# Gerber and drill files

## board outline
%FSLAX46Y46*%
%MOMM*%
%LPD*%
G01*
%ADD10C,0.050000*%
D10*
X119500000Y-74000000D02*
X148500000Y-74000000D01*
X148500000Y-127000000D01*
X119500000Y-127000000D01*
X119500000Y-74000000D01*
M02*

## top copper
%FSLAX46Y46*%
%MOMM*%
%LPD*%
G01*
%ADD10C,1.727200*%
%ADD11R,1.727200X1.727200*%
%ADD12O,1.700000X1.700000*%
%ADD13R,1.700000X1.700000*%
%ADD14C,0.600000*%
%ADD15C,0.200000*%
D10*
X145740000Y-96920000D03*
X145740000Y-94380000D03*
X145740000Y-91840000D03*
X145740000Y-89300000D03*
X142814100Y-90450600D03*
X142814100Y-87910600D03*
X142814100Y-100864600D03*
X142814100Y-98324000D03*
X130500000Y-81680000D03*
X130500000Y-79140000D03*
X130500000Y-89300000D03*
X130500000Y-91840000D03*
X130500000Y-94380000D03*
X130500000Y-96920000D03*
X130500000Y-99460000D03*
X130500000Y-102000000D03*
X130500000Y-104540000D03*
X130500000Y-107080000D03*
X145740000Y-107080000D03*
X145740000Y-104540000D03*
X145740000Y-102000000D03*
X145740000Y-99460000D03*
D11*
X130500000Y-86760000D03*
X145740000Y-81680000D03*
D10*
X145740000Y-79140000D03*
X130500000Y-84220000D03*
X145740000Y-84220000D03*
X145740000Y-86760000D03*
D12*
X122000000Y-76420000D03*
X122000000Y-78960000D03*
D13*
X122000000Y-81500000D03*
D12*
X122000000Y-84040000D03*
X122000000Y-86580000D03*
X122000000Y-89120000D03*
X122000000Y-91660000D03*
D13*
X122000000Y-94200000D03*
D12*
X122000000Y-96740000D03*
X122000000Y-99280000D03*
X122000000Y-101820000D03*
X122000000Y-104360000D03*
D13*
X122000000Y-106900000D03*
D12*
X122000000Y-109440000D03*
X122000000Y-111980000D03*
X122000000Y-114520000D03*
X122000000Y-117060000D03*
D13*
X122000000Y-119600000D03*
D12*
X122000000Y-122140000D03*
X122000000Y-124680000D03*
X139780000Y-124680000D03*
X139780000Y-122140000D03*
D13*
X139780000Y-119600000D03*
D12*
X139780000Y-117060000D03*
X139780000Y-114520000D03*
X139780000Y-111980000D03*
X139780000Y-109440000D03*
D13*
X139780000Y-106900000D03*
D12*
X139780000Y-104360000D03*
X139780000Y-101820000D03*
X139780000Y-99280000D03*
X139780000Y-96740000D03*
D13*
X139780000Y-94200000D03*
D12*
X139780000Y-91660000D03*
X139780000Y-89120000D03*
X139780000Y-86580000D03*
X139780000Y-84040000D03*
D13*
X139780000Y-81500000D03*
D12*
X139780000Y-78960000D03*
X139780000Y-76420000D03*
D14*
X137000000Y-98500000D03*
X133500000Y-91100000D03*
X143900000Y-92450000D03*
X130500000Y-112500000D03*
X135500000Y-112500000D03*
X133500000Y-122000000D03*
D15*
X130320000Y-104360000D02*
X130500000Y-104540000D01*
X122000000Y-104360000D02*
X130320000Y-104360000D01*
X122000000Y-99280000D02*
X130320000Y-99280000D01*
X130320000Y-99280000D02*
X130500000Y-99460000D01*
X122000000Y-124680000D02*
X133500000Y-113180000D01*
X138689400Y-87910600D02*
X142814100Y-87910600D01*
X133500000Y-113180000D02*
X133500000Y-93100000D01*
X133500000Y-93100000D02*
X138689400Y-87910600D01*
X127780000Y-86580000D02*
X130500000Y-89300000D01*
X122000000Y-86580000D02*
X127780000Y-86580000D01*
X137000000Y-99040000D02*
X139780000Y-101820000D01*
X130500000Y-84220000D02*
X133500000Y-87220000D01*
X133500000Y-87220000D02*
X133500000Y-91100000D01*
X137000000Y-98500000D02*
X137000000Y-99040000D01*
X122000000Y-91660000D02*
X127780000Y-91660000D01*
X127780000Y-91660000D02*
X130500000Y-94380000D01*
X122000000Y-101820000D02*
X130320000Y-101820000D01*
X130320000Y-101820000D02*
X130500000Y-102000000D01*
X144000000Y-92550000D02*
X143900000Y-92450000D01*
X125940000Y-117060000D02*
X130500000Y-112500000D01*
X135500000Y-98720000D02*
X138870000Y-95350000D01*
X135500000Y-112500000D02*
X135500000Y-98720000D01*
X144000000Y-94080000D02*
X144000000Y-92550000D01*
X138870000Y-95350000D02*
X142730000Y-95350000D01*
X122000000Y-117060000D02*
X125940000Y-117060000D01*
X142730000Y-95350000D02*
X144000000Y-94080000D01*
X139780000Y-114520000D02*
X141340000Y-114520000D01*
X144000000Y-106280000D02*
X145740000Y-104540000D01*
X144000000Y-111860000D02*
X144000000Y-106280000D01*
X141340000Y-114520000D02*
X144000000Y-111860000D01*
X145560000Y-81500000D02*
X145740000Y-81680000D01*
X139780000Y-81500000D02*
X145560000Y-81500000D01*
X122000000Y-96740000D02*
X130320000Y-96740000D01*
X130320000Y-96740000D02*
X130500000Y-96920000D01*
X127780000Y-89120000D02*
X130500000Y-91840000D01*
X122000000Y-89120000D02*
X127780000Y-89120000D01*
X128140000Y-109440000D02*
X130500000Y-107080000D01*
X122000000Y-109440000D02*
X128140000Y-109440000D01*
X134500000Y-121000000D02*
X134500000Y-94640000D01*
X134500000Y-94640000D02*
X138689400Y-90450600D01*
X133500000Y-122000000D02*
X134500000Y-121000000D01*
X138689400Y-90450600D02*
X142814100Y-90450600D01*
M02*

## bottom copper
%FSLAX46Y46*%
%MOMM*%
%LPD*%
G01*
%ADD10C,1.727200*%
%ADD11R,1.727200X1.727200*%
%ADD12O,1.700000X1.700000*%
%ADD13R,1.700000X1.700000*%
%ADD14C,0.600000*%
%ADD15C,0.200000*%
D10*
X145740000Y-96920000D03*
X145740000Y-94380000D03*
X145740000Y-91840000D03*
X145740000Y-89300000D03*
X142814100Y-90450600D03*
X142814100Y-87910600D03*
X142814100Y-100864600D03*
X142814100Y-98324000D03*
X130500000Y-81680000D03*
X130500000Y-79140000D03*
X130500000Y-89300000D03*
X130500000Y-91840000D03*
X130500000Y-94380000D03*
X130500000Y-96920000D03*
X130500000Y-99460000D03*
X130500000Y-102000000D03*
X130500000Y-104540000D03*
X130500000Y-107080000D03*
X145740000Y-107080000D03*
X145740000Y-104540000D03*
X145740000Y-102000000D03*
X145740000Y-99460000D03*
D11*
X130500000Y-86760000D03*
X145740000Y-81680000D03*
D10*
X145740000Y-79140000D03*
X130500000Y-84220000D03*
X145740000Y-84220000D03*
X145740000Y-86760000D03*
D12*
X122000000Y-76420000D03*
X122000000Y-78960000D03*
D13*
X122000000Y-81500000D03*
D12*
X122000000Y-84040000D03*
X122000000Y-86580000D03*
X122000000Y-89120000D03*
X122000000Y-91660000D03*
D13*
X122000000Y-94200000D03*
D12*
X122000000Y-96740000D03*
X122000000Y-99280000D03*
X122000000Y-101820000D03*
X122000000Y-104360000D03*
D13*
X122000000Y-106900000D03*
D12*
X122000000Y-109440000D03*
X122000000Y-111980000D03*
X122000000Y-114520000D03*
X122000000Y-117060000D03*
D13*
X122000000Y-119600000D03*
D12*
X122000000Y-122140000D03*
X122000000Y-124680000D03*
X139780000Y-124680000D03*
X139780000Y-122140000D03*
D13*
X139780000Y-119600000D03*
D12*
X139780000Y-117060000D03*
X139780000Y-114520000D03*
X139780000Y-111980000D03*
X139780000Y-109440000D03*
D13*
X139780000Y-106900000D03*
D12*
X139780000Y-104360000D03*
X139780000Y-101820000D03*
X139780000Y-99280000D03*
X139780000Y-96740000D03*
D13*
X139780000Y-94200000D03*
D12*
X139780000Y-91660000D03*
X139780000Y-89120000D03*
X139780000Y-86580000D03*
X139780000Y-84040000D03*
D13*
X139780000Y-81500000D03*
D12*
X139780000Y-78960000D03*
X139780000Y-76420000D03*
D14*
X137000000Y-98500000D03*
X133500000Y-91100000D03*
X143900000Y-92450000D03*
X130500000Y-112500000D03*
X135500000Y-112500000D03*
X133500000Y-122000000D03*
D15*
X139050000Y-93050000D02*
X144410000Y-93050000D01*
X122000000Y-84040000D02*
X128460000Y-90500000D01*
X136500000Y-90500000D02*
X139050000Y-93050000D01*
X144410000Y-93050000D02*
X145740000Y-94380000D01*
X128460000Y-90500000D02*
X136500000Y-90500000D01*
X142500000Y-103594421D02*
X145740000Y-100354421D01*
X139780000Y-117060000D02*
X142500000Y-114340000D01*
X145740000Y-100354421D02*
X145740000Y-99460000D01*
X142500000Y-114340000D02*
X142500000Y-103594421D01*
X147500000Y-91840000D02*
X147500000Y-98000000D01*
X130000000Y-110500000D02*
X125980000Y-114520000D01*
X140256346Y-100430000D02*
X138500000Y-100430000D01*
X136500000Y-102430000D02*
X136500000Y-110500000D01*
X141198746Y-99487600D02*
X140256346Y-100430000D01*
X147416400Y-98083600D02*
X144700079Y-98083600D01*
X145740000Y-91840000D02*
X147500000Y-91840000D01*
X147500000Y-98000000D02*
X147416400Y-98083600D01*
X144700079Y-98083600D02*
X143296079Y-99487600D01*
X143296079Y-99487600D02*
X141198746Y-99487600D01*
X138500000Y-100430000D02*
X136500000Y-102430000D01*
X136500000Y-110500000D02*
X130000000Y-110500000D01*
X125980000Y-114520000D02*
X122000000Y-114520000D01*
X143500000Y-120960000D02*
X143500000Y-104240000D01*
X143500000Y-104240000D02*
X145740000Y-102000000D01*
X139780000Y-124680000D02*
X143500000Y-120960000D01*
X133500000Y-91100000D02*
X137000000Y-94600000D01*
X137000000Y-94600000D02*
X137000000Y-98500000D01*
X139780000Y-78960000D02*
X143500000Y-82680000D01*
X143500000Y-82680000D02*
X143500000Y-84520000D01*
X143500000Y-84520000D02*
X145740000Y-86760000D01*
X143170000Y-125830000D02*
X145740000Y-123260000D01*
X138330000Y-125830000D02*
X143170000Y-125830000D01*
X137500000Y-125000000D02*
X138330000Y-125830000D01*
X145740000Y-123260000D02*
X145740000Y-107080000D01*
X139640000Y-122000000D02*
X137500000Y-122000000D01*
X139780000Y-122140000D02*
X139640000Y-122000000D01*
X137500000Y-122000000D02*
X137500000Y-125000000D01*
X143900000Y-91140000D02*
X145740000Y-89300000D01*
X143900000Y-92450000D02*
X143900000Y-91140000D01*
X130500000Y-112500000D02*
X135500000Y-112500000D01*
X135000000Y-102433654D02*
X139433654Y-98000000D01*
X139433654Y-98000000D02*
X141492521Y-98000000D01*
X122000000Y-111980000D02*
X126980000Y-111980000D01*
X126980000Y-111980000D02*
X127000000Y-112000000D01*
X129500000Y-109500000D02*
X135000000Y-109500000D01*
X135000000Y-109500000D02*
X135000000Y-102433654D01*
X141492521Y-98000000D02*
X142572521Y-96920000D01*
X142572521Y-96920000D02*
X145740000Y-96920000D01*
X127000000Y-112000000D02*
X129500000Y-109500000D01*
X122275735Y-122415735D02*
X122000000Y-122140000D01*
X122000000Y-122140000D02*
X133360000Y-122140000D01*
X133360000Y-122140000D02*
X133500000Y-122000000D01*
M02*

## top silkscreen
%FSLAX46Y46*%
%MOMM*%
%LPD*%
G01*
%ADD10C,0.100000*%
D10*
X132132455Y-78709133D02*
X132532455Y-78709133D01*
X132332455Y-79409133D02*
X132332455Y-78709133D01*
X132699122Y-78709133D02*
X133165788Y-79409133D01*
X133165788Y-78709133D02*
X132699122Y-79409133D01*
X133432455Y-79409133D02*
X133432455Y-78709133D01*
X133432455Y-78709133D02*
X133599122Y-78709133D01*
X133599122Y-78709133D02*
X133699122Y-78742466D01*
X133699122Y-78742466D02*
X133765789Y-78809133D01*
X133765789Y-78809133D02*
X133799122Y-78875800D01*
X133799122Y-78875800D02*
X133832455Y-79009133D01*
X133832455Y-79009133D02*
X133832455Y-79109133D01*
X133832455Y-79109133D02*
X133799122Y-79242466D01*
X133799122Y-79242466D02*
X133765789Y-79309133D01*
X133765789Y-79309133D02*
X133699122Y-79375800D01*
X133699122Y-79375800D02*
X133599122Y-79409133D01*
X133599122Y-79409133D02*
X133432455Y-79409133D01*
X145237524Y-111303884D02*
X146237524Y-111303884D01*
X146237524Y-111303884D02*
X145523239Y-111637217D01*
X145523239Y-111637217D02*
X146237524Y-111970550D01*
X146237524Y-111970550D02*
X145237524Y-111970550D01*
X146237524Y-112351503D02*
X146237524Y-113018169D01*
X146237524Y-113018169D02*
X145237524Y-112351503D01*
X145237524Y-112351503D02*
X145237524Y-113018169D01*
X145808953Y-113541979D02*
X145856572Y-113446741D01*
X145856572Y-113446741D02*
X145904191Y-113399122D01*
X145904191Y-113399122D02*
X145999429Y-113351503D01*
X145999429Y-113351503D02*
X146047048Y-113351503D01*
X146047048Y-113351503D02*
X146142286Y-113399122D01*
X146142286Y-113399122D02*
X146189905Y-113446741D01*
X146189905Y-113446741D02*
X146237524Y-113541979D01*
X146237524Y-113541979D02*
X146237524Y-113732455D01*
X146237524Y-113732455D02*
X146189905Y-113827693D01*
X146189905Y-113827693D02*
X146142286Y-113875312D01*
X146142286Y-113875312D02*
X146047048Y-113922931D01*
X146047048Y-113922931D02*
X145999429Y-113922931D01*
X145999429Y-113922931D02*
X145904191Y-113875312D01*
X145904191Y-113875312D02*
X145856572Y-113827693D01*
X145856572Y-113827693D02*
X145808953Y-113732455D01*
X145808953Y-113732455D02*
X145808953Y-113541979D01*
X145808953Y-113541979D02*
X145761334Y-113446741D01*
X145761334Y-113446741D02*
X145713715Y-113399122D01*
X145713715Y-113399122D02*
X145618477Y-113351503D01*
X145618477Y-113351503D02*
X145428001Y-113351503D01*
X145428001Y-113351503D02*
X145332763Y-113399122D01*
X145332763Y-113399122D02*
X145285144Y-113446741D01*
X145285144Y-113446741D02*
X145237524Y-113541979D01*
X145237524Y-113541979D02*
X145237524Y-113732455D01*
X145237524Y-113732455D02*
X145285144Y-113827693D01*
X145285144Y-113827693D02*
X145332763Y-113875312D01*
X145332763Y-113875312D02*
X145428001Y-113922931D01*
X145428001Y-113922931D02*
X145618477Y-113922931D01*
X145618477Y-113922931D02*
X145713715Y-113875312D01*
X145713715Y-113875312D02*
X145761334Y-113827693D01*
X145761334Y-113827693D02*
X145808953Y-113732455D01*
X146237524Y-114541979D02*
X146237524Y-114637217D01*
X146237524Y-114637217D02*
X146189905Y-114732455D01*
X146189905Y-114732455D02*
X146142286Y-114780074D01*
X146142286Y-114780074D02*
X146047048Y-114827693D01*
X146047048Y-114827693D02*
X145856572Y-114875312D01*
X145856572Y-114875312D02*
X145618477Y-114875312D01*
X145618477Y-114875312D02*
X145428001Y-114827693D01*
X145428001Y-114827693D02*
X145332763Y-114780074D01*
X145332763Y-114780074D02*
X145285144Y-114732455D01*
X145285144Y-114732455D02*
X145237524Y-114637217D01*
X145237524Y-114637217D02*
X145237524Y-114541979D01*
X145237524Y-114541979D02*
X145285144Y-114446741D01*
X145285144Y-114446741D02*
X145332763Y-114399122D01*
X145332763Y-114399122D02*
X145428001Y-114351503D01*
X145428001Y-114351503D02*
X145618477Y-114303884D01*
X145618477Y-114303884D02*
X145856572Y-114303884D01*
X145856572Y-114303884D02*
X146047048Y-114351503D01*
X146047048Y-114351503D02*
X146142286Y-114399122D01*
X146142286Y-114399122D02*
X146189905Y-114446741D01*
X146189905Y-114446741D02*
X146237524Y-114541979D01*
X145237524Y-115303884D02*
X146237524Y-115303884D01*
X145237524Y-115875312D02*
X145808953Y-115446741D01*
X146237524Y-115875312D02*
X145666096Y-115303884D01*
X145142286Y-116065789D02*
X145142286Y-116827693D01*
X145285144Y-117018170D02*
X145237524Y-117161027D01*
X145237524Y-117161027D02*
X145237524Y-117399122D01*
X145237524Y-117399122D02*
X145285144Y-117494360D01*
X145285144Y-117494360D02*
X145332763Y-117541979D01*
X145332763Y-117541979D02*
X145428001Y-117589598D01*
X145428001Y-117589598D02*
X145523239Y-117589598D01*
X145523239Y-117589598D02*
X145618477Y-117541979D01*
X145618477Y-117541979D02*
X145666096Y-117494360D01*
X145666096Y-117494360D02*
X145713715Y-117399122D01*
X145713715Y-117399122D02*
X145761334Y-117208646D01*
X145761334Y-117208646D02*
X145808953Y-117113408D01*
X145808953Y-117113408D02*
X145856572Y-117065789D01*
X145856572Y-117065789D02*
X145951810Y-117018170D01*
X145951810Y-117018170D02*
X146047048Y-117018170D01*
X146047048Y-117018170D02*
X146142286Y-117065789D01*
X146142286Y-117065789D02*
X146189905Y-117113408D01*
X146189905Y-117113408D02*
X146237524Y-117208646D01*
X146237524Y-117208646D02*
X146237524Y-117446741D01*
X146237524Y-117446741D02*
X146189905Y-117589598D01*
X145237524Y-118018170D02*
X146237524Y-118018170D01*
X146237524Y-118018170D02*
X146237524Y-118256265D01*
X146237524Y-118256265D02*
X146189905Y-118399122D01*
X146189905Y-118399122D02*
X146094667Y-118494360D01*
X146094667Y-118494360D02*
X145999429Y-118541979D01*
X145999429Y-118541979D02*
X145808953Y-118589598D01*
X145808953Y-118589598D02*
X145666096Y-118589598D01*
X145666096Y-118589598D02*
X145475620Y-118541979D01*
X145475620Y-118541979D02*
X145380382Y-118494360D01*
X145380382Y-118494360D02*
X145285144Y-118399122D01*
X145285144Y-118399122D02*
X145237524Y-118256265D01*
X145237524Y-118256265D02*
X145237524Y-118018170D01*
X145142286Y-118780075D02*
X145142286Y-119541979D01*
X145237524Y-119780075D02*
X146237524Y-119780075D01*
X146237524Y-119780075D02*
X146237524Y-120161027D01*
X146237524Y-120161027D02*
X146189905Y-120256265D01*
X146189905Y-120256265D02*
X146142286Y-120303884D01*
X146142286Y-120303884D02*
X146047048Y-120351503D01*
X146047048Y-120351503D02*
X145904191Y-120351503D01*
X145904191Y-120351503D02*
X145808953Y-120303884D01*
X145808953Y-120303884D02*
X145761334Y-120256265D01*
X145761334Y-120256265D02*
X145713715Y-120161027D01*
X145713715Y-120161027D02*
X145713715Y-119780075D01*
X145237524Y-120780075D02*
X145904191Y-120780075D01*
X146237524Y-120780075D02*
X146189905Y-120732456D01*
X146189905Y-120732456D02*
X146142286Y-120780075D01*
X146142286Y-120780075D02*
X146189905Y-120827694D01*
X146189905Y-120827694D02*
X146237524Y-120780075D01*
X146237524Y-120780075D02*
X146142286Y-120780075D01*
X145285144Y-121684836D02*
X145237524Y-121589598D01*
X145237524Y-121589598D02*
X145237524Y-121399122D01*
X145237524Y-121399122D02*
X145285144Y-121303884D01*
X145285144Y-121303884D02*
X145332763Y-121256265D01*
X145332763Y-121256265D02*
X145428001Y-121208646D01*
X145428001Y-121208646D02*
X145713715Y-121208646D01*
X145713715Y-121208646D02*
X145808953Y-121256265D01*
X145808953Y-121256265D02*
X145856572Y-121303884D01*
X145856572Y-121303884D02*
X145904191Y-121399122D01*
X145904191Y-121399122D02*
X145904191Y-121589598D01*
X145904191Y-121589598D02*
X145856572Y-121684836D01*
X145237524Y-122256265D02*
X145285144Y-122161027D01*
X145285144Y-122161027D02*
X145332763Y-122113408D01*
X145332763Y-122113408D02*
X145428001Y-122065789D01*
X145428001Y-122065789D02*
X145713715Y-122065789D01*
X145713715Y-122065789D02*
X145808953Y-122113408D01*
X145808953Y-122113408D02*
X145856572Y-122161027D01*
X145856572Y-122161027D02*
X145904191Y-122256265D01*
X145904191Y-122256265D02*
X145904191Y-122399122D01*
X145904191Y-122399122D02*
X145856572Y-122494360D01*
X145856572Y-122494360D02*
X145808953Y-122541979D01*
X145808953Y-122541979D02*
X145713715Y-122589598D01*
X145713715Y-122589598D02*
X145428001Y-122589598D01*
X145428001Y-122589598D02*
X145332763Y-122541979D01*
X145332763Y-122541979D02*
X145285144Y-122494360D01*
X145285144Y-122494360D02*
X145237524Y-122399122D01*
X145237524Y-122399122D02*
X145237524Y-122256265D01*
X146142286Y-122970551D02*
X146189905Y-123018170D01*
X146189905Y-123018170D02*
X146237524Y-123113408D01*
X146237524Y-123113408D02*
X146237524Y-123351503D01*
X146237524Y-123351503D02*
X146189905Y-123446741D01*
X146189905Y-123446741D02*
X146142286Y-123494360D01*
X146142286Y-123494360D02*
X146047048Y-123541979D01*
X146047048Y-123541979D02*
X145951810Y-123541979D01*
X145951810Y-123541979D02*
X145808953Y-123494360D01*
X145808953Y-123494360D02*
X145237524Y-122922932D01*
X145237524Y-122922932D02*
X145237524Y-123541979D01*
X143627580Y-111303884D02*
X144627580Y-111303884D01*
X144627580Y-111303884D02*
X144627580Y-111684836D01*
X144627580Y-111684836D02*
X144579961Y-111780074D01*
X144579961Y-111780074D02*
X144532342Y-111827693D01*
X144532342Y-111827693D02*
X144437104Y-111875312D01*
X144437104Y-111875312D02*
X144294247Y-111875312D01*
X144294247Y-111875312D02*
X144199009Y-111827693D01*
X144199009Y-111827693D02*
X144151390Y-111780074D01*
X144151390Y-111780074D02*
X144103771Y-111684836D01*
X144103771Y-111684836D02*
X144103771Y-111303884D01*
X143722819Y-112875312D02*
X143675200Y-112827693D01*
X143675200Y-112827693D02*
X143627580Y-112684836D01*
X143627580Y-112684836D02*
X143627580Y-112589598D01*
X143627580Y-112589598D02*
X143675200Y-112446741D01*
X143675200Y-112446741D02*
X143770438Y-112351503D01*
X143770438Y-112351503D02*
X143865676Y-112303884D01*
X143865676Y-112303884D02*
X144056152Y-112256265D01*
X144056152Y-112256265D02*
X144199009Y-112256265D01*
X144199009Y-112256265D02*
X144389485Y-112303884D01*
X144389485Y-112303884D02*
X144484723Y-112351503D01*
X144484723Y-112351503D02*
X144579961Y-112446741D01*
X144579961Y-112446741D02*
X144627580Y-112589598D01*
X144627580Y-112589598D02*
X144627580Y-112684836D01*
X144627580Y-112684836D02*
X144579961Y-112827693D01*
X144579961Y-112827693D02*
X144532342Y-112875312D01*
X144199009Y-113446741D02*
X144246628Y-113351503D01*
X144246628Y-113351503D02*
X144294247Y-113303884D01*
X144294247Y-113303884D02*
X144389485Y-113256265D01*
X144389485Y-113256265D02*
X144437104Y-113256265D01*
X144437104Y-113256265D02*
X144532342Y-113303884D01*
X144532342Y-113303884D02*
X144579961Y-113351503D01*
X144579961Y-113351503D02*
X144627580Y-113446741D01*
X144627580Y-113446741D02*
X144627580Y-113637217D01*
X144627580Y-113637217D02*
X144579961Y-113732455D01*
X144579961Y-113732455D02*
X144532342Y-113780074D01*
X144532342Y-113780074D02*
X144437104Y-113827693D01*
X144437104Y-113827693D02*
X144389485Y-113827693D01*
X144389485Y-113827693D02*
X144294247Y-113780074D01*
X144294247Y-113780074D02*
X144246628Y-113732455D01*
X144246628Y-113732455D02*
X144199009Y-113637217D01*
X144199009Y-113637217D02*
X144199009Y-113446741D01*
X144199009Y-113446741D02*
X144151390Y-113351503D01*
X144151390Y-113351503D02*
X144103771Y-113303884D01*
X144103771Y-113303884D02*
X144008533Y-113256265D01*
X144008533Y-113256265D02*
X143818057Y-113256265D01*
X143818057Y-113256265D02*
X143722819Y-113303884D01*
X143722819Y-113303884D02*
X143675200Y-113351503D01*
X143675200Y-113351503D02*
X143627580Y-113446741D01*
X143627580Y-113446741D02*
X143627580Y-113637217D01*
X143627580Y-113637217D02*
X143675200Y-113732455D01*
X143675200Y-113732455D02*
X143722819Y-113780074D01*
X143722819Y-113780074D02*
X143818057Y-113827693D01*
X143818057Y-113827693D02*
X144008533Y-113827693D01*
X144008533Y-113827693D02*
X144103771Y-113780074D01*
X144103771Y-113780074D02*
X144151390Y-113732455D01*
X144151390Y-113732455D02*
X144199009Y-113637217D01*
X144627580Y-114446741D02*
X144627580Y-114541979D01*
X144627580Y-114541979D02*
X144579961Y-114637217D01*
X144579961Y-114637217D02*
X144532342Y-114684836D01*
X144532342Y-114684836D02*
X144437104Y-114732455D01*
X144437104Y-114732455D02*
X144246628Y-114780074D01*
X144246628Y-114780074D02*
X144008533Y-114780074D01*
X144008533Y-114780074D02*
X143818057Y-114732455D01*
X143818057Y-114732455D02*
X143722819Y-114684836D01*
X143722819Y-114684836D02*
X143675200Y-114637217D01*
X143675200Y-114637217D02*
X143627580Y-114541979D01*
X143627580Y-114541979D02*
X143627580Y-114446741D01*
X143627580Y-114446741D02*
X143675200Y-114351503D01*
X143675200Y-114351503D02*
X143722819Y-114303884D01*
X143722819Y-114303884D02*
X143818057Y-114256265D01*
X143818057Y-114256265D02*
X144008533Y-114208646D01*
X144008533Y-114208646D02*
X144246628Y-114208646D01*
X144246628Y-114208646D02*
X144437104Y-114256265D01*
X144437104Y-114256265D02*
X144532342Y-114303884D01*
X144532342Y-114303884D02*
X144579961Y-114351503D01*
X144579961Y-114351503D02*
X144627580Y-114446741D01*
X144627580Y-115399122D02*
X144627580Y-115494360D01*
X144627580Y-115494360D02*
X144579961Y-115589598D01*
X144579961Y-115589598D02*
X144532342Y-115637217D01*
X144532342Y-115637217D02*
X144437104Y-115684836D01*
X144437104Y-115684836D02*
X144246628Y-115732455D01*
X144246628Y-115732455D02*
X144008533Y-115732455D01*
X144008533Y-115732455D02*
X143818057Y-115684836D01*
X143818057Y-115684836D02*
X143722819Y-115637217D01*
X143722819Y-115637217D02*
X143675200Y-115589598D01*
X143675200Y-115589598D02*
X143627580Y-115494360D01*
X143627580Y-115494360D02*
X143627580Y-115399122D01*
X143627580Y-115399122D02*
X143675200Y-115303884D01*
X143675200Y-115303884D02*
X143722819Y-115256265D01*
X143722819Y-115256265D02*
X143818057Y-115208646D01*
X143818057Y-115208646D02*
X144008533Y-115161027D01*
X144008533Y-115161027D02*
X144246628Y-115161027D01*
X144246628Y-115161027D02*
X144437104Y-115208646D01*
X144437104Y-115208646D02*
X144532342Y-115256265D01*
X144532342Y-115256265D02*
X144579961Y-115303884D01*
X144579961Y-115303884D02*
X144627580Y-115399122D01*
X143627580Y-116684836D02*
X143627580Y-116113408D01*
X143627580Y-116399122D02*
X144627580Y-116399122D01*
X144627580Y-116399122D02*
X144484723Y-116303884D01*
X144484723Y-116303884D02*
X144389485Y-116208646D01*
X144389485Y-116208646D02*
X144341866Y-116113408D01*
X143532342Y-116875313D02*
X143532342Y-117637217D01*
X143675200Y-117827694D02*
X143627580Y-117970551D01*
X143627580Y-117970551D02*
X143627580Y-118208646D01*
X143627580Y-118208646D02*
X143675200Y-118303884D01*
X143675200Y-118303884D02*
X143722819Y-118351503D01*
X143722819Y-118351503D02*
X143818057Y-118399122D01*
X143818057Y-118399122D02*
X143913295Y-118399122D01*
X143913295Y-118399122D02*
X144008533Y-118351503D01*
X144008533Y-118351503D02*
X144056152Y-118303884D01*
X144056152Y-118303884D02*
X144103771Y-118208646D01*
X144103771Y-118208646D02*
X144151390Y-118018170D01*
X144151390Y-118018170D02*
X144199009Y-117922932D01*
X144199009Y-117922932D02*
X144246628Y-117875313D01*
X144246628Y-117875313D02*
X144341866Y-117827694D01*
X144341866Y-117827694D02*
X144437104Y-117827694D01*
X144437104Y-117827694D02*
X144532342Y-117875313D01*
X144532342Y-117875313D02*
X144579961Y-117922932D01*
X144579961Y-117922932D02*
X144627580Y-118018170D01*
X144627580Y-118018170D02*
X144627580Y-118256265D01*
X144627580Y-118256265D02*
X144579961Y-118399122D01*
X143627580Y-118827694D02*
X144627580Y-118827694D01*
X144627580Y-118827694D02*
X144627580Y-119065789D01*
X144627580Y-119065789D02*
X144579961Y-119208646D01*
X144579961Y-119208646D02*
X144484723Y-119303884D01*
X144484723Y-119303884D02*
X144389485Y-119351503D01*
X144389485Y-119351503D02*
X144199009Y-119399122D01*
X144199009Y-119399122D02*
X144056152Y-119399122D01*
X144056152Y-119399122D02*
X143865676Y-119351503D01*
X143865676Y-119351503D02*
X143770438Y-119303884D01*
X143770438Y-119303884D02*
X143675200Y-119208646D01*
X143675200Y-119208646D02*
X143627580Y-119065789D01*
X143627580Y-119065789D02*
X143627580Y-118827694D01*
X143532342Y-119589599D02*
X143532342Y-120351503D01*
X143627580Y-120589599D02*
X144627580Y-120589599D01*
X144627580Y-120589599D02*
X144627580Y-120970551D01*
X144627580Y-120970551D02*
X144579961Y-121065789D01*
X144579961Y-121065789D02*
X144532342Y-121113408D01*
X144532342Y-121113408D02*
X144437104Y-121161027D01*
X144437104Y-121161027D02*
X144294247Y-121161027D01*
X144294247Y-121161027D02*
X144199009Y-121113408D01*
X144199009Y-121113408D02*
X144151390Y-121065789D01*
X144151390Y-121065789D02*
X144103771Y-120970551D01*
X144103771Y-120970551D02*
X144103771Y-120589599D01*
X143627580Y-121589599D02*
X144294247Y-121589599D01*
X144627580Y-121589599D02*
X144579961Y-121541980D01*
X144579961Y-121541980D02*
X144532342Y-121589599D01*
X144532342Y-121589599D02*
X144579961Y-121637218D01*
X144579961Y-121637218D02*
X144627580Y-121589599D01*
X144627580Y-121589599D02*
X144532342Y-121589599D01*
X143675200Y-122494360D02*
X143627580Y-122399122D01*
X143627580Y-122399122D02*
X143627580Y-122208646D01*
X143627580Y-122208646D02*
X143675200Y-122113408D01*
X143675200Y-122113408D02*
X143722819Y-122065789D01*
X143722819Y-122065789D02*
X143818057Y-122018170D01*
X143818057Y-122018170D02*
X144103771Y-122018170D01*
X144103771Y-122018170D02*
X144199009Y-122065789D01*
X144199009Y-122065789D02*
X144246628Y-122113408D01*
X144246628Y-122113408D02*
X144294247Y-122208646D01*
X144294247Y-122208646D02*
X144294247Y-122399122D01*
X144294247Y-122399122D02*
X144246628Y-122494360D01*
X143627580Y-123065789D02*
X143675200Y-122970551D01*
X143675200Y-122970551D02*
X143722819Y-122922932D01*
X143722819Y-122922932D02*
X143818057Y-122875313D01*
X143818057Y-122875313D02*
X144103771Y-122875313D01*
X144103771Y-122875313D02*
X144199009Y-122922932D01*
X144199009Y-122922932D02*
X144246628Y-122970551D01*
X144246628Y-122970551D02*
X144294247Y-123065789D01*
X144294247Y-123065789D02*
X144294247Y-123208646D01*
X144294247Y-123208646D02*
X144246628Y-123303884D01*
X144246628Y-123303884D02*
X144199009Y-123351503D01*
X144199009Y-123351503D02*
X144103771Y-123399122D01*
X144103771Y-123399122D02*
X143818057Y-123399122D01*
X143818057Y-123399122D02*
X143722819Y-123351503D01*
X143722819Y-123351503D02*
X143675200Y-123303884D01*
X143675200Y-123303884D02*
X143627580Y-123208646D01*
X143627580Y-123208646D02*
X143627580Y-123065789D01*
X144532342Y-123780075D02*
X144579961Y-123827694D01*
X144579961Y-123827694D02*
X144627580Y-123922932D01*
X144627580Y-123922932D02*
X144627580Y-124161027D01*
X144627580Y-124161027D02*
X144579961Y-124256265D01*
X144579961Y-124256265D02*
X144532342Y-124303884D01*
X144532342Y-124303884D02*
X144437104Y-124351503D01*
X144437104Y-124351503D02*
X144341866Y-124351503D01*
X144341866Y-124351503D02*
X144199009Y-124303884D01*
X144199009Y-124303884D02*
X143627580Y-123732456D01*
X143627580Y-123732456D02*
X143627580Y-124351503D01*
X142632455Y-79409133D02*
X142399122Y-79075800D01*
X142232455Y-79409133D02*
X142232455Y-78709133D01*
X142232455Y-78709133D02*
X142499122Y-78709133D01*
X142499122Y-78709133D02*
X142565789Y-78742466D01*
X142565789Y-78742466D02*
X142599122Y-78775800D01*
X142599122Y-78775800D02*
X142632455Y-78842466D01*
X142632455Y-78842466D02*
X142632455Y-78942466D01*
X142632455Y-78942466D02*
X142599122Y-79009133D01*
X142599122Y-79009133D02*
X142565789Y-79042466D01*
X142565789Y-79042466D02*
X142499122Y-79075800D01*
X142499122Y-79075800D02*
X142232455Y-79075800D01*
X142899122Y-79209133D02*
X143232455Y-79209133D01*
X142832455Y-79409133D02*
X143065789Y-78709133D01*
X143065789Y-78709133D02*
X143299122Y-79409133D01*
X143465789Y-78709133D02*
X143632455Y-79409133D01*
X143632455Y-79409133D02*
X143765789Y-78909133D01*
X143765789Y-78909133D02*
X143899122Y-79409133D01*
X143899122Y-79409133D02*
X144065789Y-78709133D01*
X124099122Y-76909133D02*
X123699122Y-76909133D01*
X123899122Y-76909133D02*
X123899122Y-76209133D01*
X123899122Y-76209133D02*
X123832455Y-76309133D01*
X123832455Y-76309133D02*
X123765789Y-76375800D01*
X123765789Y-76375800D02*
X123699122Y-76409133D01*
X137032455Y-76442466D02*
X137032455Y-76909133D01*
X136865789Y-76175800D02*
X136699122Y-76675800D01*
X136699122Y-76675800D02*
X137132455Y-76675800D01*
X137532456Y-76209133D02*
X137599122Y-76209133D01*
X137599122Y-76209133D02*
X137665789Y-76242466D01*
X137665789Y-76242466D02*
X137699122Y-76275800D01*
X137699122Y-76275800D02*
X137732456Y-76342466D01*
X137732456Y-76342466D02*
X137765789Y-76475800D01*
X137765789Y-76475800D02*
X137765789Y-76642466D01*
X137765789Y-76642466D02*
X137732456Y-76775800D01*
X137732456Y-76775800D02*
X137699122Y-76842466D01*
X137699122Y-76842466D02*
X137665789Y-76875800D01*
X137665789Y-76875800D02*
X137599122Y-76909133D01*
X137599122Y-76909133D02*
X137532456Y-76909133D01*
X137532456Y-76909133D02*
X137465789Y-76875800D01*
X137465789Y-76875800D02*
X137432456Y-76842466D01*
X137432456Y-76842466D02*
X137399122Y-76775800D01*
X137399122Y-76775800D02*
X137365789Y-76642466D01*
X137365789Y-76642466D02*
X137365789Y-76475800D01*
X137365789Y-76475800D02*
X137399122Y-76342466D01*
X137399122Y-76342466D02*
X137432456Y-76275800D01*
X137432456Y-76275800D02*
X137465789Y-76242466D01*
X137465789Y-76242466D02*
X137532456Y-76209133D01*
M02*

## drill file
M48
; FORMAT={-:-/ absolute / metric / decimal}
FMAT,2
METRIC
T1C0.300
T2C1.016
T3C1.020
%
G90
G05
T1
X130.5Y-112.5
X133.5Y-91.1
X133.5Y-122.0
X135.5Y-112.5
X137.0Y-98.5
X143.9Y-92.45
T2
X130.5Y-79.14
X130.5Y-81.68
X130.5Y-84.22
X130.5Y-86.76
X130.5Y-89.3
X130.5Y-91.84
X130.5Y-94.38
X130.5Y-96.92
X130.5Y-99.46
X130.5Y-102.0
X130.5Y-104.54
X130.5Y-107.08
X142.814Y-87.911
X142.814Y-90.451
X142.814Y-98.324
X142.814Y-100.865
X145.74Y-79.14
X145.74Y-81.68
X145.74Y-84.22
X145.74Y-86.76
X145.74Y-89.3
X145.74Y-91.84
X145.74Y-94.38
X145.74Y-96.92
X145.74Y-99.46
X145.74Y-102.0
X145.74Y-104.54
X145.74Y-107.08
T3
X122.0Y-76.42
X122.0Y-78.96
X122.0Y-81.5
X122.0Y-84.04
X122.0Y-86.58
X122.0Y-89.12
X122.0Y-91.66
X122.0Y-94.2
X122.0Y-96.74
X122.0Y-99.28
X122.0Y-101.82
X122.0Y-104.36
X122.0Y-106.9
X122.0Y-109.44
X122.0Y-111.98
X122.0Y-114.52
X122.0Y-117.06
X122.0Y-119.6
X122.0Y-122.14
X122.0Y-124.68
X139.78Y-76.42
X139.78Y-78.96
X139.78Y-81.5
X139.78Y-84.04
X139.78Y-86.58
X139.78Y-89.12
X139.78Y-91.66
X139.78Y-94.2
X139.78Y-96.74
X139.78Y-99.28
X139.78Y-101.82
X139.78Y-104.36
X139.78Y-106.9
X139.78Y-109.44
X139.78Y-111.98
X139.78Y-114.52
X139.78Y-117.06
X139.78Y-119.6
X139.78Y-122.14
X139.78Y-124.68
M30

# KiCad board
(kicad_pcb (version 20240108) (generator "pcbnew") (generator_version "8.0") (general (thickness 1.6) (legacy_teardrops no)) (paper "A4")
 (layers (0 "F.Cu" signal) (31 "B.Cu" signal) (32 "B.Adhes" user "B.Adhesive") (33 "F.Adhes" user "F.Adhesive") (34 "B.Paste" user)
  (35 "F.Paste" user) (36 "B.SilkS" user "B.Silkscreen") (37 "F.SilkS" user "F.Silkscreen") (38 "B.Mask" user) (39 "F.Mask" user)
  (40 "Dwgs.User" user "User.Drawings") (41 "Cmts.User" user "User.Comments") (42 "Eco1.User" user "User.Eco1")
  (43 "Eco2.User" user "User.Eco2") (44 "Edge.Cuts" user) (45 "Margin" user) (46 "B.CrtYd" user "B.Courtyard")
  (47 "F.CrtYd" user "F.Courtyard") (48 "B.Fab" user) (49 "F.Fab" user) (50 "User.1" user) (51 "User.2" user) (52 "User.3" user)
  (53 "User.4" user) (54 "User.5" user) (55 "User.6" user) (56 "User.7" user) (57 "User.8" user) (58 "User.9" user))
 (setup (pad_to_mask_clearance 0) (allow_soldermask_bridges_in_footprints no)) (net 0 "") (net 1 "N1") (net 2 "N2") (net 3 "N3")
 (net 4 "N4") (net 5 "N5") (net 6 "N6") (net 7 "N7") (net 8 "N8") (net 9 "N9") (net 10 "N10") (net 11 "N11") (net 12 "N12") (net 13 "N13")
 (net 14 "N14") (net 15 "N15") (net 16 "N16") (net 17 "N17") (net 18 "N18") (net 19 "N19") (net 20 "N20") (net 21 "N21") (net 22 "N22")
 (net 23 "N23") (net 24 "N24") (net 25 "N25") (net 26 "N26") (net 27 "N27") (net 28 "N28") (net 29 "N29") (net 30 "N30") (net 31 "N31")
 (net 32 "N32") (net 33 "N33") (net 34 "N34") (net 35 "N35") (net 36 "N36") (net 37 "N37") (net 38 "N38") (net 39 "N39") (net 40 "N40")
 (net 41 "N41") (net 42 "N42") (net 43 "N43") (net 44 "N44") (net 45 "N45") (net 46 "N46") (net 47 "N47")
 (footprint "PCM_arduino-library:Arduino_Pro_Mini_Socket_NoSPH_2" (layer "F.Cu") (at 138.12 91.84)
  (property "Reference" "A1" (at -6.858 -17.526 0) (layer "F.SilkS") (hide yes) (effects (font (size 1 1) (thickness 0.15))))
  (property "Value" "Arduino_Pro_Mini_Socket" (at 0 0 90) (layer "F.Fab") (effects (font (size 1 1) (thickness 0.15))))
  (pad "A0" thru_hole circle (at 7.62 5.08) (size 1.7272 1.7272) (drill 1.016) (layers "*.Cu" "*.Mask") (remove_unused_layers no)
   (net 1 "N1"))
  (pad "A1" thru_hole circle (at 7.62 2.54) (size 1.7272 1.7272) (drill 1.016) (layers "*.Cu" "*.Mask") (remove_unused_layers no)
   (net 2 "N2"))
  (pad "A2" thru_hole circle (at 7.62 0) (size 1.7272 1.7272) (drill 1.016) (layers "*.Cu" "*.Mask") (remove_unused_layers no) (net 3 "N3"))
  (pad "A3" thru_hole circle (at 7.62 -2.54) (size 1.7272 1.7272) (drill 1.016) (layers "*.Cu" "*.Mask") (remove_unused_layers no)
   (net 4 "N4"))
  (pad "A4" thru_hole circle (at 4.6941 -1.3894) (size 1.7272 1.7272) (drill 1.016) (layers "*.Cu" "*.Mask") (remove_unused_layers no)
   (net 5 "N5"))
  (pad "A5" thru_hole circle (at 4.6941 -3.9294) (size 1.7272 1.7272) (drill 1.016) (layers "*.Cu" "*.Mask") (remove_unused_layers no)
   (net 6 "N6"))
  (pad "A6" thru_hole circle (at 4.6941 9.0246) (size 1.7272 1.7272) (drill 1.016) (layers "*.Cu" "*.Mask") (remove_unused_layers no)
   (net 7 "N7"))
  (pad "A7" thru_hole circle (at 4.6941 6.484) (size 1.7272 1.7272) (drill 1.016) (layers "*.Cu" "*.Mask") (remove_unused_layers no)
   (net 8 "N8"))
  (pad "D0" thru_hole circle (at -7.62 -10.16) (size 1.7272 1.7272) (drill 1.016) (layers "*.Cu" "*.Mask") (remove_unused_layers no)
   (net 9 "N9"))
  (pad "D1" thru_hole circle (at -7.62 -12.7) (size 1.7272 1.7272) (drill 1.016) (layers "*.Cu" "*.Mask") (remove_unused_layers no)
   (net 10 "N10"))
  (pad "D2" thru_hole circle (at -7.62 -2.54) (size 1.7272 1.7272) (drill 1.016) (layers "*.Cu" "*.Mask") (remove_unused_layers no)
   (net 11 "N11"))
  (pad "D3" thru_hole circle (at -7.62 0) (size 1.7272 1.7272) (drill 1.016) (layers "*.Cu" "*.Mask") (remove_unused_layers no)
   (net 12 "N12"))
  (pad "D4" thru_hole circle (at -7.62 2.54) (size 1.7272 1.7272) (drill 1.016) (layers "*.Cu" "*.Mask") (remove_unused_layers no)
   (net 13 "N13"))
  (pad "D5" thru_hole circle (at -7.62 5.08) (size 1.7272 1.7272) (drill 1.016) (layers "*.Cu" "*.Mask") (remove_unused_layers no)
   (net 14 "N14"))
  (pad "D6" thru_hole circle (at -7.62 7.62) (size 1.7272 1.7272) (drill 1.016) (layers "*.Cu" "*.Mask") (remove_unused_layers no)
   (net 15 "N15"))
  (pad "D7" thru_hole circle (at -7.62 10.16) (size 1.7272 1.7272) (drill 1.016) (layers "*.Cu" "*.Mask") (remove_unused_layers no)
   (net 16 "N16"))
  (pad "D8" thru_hole circle (at -7.62 12.7) (size 1.7272 1.7272) (drill 1.016) (layers "*.Cu" "*.Mask") (remove_unused_layers no)
   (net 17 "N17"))
  (pad "D9" thru_hole circle (at -7.62 15.24) (size 1.7272 1.7272) (drill 1.016) (layers "*.Cu" "*.Mask") (remove_unused_layers no)
   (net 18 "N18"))
  (pad "D10" thru_hole circle (at 7.62 15.24) (size 1.7272 1.7272) (drill 1.016) (layers "*.Cu" "*.Mask") (remove_unused_layers no)
   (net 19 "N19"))
  (pad "D11" thru_hole circle (at 7.62 12.7) (size 1.7272 1.7272) (drill 1.016) (layers "*.Cu" "*.Mask") (remove_unused_layers no)
   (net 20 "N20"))
  (pad "D12" thru_hole circle (at 7.62 10.16) (size 1.7272 1.7272) (drill 1.016) (layers "*.Cu" "*.Mask") (remove_unused_layers no)
   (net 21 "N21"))
  (pad "D13" thru_hole circle (at 7.62 7.62) (size 1.7272 1.7272) (drill 1.016) (layers "*.Cu" "*.Mask") (remove_unused_layers no)
   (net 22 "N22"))
  (pad "GND1" thru_hole rect (at -7.62 -5.08) (size 1.7272 1.7272) (drill 1.016) (layers "*.Cu" "*.Mask") (remove_unused_layers no)
   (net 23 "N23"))
  (pad "GND2" thru_hole rect (at 7.62 -10.16) (size 1.7272 1.7272) (drill 1.016) (layers "*.Cu" "*.Mask") (remove_unused_layers no)
   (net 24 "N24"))
  (pad "RAW" thru_hole circle (at 7.62 -12.7) (size 1.7272 1.7272) (drill 1.016) (layers "*.Cu" "*.Mask") (remove_unused_layers no)
   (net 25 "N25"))
  (pad "RST1" thru_hole circle (at -7.62 -7.62) (size 1.7272 1.7272) (drill 1.016) (layers "*.Cu" "*.Mask") (remove_unused_layers no)
   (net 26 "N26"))
  (pad "RST2" thru_hole circle (at 7.62 -7.62) (size 1.7272 1.7272) (drill 1.016) (layers "*.Cu" "*.Mask") (remove_unused_layers no)
   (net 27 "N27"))
  (pad "Vcc1" thru_hole circle (at 7.62 -5.08) (size 1.7272 1.7272) (drill 1.016) (layers "*.Cu" "*.Mask") (remove_unused_layers no)
   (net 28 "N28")))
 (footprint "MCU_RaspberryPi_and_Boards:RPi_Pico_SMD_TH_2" (layer "F.Cu") (at 130.89 100.55)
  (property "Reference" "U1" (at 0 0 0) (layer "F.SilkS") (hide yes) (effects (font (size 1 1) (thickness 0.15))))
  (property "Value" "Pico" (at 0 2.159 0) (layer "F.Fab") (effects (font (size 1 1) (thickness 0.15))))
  (pad "1" thru_hole oval (at -8.89 -24.13) (size 1.7 1.7) (drill 1.02) (layers "*.Cu" "*.Mask") (remove_unused_layers no) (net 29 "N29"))
  (pad "2" thru_hole oval (at -8.89 -21.59) (size 1.7 1.7) (drill 1.02) (layers "*.Cu" "*.Mask") (remove_unused_layers no) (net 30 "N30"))
  (pad "3" thru_hole rect (at -8.89 -19.05) (size 1.7 1.7) (drill 1.02) (layers "*.Cu" "*.Mask") (remove_unused_layers no) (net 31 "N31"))
  (pad "4" thru_hole oval (at -8.89 -16.51) (size 1.7 1.7) (drill 1.02) (layers "*.Cu" "*.Mask") (remove_unused_layers no) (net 2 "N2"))
  (pad "5" thru_hole oval (at -8.89 -13.97) (size 1.7 1.7) (drill 1.02) (layers "*.Cu" "*.Mask") (remove_unused_layers no) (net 11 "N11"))
  (pad "6" thru_hole oval (at -8.89 -11.43) (size 1.7 1.7) (drill 1.02) (layers "*.Cu" "*.Mask") (remove_unused_layers no) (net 12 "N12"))
  (pad "7" thru_hole oval (at -8.89 -8.89) (size 1.7 1.7) (drill 1.02) (layers "*.Cu" "*.Mask") (remove_unused_layers no) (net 13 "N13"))
  (pad "8" thru_hole rect (at -8.89 -6.35) (size 1.7 1.7) (drill 1.02) (layers "*.Cu" "*.Mask") (remove_unused_layers no) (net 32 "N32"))
  (pad "9" thru_hole oval (at -8.89 -3.81) (size 1.7 1.7) (drill 1.02) (layers "*.Cu" "*.Mask") (remove_unused_layers no) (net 14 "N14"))
  (pad "10" thru_hole oval (at -8.89 -1.27) (size 1.7 1.7) (drill 1.02) (layers "*.Cu" "*.Mask") (remove_unused_layers no) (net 15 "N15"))
  (pad "11" thru_hole oval (at -8.89 1.27) (size 1.7 1.7) (drill 1.02) (layers "*.Cu" "*.Mask") (remove_unused_layers no) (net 16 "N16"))
  (pad "12" thru_hole oval (at -8.89 3.81) (size 1.7 1.7) (drill 1.02) (layers "*.Cu" "*.Mask") (remove_unused_layers no) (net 17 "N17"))
  (pad "13" thru_hole rect (at -8.89 6.35) (size 1.7 1.7) (drill 1.02) (layers "*.Cu" "*.Mask") (remove_unused_layers no) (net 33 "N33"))
  (pad "14" thru_hole oval (at -8.89 8.89) (size 1.7 1.7) (drill 1.02) (layers "*.Cu" "*.Mask") (remove_unused_layers no) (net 18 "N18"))
  (pad "15" thru_hole oval (at -8.89 11.43) (size 1.7 1.7) (drill 1.02) (layers "*.Cu" "*.Mask") (remove_unused_layers no) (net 1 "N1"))
  (pad "16" thru_hole oval (at -8.89 13.97) (size 1.7 1.7) (drill 1.02) (layers "*.Cu" "*.Mask") (remove_unused_layers no) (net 3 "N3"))
  (pad "17" thru_hole oval (at -8.89 16.51) (size 1.7 1.7) (drill 1.02) (layers "*.Cu" "*.Mask") (remove_unused_layers no) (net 4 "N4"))
  (pad "18" thru_hole rect (at -8.89 19.05) (size 1.7 1.7) (drill 1.02) (layers "*.Cu" "*.Mask") (remove_unused_layers no) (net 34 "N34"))
  (pad "19" thru_hole oval (at -8.89 21.59) (size 1.7 1.7) (drill 1.02) (layers "*.Cu" "*.Mask") (remove_unused_layers no) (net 5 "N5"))
  (pad "20" thru_hole oval (at -8.89 24.13) (size 1.7 1.7) (drill 1.02) (layers "*.Cu" "*.Mask") (remove_unused_layers no) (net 6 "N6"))
  (pad "21" thru_hole oval (at 8.89 24.13) (size 1.7 1.7) (drill 1.02) (layers "*.Cu" "*.Mask") (remove_unused_layers no) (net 21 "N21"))
  (pad "22" thru_hole oval (at 8.89 21.59) (size 1.7 1.7) (drill 1.02) (layers "*.Cu" "*.Mask") (remove_unused_layers no) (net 19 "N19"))
  (pad "23" thru_hole rect (at 8.89 19.05) (size 1.7 1.7) (drill 1.02) (layers "*.Cu" "*.Mask") (remove_unused_layers no) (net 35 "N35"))
  (pad "24" thru_hole oval (at 8.89 16.51) (size 1.7 1.7) (drill 1.02) (layers "*.Cu" "*.Mask") (remove_unused_layers no) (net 22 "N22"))
  (pad "25" thru_hole oval (at 8.89 13.97) (size 1.7 1.7) (drill 1.02) (layers "*.Cu" "*.Mask") (remove_unused_layers no) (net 20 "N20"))
  (pad "26" thru_hole oval (at 8.89 11.43) (size 1.7 1.7) (drill 1.02) (layers "*.Cu" "*.Mask") (remove_unused_layers no) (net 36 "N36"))
  (pad "27" thru_hole oval (at 8.89 8.89) (size 1.7 1.7) (drill 1.02) (layers "*.Cu" "*.Mask") (remove_unused_layers no) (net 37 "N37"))
  (pad "28" thru_hole rect (at 8.89 6.35) (size 1.7 1.7) (drill 1.02) (layers "*.Cu" "*.Mask") (remove_unused_layers no) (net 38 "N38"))
  (pad "29" thru_hole oval (at 8.89 3.81) (size 1.7 1.7) (drill 1.02) (layers "*.Cu" "*.Mask") (remove_unused_layers no) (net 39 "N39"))
  (pad "30" thru_hole oval (at 8.89 1.27) (size 1.7 1.7) (drill 1.02) (layers "*.Cu" "*.Mask") (remove_unused_layers no) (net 26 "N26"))
  (pad "31" thru_hole oval (at 8.89 -1.27) (size 1.7 1.7) (drill 1.02) (layers "*.Cu" "*.Mask") (remove_unused_layers no) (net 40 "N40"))
  (pad "32" thru_hole oval (at 8.89 -3.81) (size 1.7 1.7) (drill 1.02) (layers "*.Cu" "*.Mask") (remove_unused_layers no) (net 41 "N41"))
  (pad "33" thru_hole rect (at 8.89 -6.35) (size 1.7 1.7) (drill 1.02) (layers "*.Cu" "*.Mask") (remove_unused_layers no) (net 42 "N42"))
  (pad "34" thru_hole oval (at 8.89 -8.89) (size 1.7 1.7) (drill 1.02) (layers "*.Cu" "*.Mask") (remove_unused_layers no) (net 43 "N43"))
  (pad "35" thru_hole oval (at 8.89 -11.43) (size 1.7 1.7) (drill 1.02) (layers "*.Cu" "*.Mask") (remove_unused_layers no) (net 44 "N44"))
  (pad "36" thru_hole oval (at 8.89 -13.97) (size 1.7 1.7) (drill 1.02) (layers "*.Cu" "*.Mask") (remove_unused_layers no) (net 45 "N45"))
  (pad "37" thru_hole oval (at 8.89 -16.51) (size 1.7 1.7) (drill 1.02) (layers "*.Cu" "*.Mask") (remove_unused_layers no) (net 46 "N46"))
  (pad "38" thru_hole rect (at 8.89 -19.05) (size 1.7 1.7) (drill 1.02) (layers "*.Cu" "*.Mask") (remove_unused_layers no) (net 24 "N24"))
  (pad "39" thru_hole oval (at 8.89 -21.59) (size 1.7 1.7) (drill 1.02) (layers "*.Cu" "*.Mask") (remove_unused_layers no) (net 28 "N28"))
  (pad "40" thru_hole oval (at 8.89 -24.13) (size 1.7 1.7) (drill 1.02) (layers "*.Cu" "*.Mask") (remove_unused_layers no) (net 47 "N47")))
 (gr_rect (start 119.5 74) (end 148.5 127) (stroke (width 0.05) (type default)) (fill none) (layer "Edge.Cuts"))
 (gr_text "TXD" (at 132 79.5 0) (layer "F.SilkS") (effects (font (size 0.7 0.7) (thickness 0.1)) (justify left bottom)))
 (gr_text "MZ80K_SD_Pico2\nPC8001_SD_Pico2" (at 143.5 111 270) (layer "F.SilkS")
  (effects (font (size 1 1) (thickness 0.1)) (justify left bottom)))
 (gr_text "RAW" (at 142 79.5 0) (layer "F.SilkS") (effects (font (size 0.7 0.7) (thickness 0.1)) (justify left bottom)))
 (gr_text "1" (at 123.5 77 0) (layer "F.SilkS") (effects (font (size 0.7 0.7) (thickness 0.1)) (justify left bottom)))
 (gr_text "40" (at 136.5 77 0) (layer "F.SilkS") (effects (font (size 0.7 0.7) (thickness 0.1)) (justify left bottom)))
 (segment (start 139.05 93.05) (end 144.41 93.05) (width 0.2) (layer "B.Cu") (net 2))
 (segment (start 122 84.04) (end 128.46 90.5) (width 0.2) (layer "B.Cu") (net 2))
 (segment (start 136.5 90.5) (end 139.05 93.05) (width 0.2) (layer "B.Cu") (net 2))
 (segment (start 144.41 93.05) (end 145.74 94.38) (width 0.2) (layer "B.Cu") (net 2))
 (segment (start 128.46 90.5) (end 136.5 90.5) (width 0.2) (layer "B.Cu") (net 2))
 (segment (start 130.32 104.36) (end 130.5 104.54) (width 0.2) (layer "F.Cu") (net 17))
 (segment (start 122 104.36) (end 130.32 104.36) (width 0.2) (layer "F.Cu") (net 17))
 (segment (start 122 99.28) (end 130.32 99.28) (width 0.2) (layer "F.Cu") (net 15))
 (segment (start 130.32 99.28) (end 130.5 99.46) (width 0.2) (layer "F.Cu") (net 15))
 (segment (start 142.5 103.594421) (end 145.74 100.354421) (width 0.2) (layer "B.Cu") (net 22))
 (segment (start 139.78 117.06) (end 142.5 114.34) (width 0.2) (layer "B.Cu") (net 22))
 (segment (start 145.74 100.354421) (end 145.74 99.46) (width 0.2) (layer "B.Cu") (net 22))
 (segment (start 142.5 114.34) (end 142.5 103.594421) (width 0.2) (layer "B.Cu") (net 22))
 (segment (start 147.5 91.84) (end 147.5 98) (width 0.2) (layer "B.Cu") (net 3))
 (segment (start 130 110.5) (end 125.98 114.52) (width 0.2) (layer "B.Cu") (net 3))
 (segment (start 140.256346 100.43) (end 138.5 100.43) (width 0.2) (layer "B.Cu") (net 3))
 (segment (start 136.5 102.43) (end 136.5 110.5) (width 0.2) (layer "B.Cu") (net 3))
 (segment (start 141.198746 99.4876) (end 140.256346 100.43) (width 0.2) (layer "B.Cu") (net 3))
 (segment (start 147.4164 98.0836) (end 144.700079 98.0836) (width 0.2) (layer "B.Cu") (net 3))
 (segment (start 145.74 91.84) (end 147.5 91.84) (width 0.2) (layer "B.Cu") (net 3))
 (segment (start 147.5 98) (end 147.4164 98.0836) (width 0.2) (layer "B.Cu") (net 3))
 (segment (start 144.700079 98.0836) (end 143.296079 99.4876) (width 0.2) (layer "B.Cu") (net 3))
 (segment (start 143.296079 99.4876) (end 141.198746 99.4876) (width 0.2) (layer "B.Cu") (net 3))
 (segment (start 138.5 100.43) (end 136.5 102.43) (width 0.2) (layer "B.Cu") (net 3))
 (segment (start 136.5 110.5) (end 130 110.5) (width 0.2) (layer "B.Cu") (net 3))
 (segment (start 125.98 114.52) (end 122 114.52) (width 0.2) (layer "B.Cu") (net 3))
 (segment (start 122 124.68) (end 133.5 113.18) (width 0.2) (layer "F.Cu") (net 6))
 (segment (start 138.6894 87.9106) (end 142.8141 87.9106) (width 0.2) (layer "F.Cu") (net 6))
 (segment (start 133.5 113.18) (end 133.5 93.1) (width 0.2) (layer "F.Cu") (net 6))
 (segment (start 133.5 93.1) (end 138.6894 87.9106) (width 0.2) (layer "F.Cu") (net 6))
 (segment (start 143.5 120.96) (end 143.5 104.24) (width 0.2) (layer "B.Cu") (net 21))
 (segment (start 143.5 104.24) (end 145.74 102) (width 0.2) (layer "B.Cu") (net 21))
 (segment (start 139.78 124.68) (end 143.5 120.96) (width 0.2) (layer "B.Cu") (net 21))
 (segment (start 127.78 86.58) (end 130.5 89.3) (width 0.2) (layer "F.Cu") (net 11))
 (segment (start 122 86.58) (end 127.78 86.58) (width 0.2) (layer "F.Cu") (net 11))
 (segment (start 137 99.04) (end 139.78 101.82) (width 0.2) (layer "F.Cu") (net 26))
 (segment (start 130.5 84.22) (end 133.5 87.22) (width 0.2) (layer "F.Cu") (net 26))
 (segment (start 133.5 87.22) (end 133.5 91.1) (width 0.2) (layer "F.Cu") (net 26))
 (segment (start 137 98.5) (end 137 99.04) (width 0.2) (layer "F.Cu") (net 26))
 (via (at 137 98.5) (size 0.6) (drill 0.3) (layers "F.Cu" "B.Cu") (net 26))
 (via (at 133.5 91.1) (size 0.6) (drill 0.3) (layers "F.Cu" "B.Cu") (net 26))
 (segment (start 133.5 91.1) (end 137 94.6) (width 0.2) (layer "B.Cu") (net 26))
 (segment (start 137 94.6) (end 137 98.5) (width 0.2) (layer "B.Cu") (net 26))
 (segment (start 139.78 78.96) (end 143.5 82.68) (width 0.2) (layer "B.Cu") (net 28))
 (segment (start 143.5 82.68) (end 143.5 84.52) (width 0.2) (layer "B.Cu") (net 28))
 (segment (start 143.5 84.52) (end 145.74 86.76) (width 0.2) (layer "B.Cu") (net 28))
 (segment (start 122 91.66) (end 127.78 91.66) (width 0.2) (layer "F.Cu") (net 13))
 (segment (start 127.78 91.66) (end 130.5 94.38) (width 0.2) (layer "F.Cu") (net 13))
 (segment (start 122 101.82) (end 130.32 101.82) (width 0.2) (layer "F.Cu") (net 16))
 (segment (start 130.32 101.82) (end 130.5 102) (width 0.2) (layer "F.Cu") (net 16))
 (segment (start 143.17 125.83) (end 145.74 123.26) (width 0.2) (layer "B.Cu") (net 19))
 (segment (start 138.33 125.83) (end 143.17 125.83) (width 0.2) (layer "B.Cu") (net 19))
 (segment (start 137.5 125) (end 138.33 125.83) (width 0.2) (layer "B.Cu") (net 19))
 (segment (start 145.74 123.26) (end 145.74 107.08) (width 0.2) (layer "B.Cu") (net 19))
 (segment (start 139.64 122) (end 137.5 122) (width 0.2) (layer "B.Cu") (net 19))
 (segment (start 139.78 122.14) (end 139.64 122) (width 0.2) (layer "B.Cu") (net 19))
 (segment (start 137.5 122) (end 137.5 125) (width 0.2) (layer "B.Cu") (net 19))
 (segment (start 144 92.55) (end 143.9 92.45) (width 0.2) (layer "F.Cu") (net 4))
 (segment (start 125.94 117.06) (end 130.5 112.5) (width 0.2) (layer "F.Cu") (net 4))
 (segment (start 135.5 98.72) (end 138.87 95.35) (width 0.2) (layer "F.Cu") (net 4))
 (segment (start 135.5 112.5) (end 135.5 98.72) (width 0.2) (layer "F.Cu") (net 4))
 (segment (start 144 94.08) (end 144 92.55) (width 0.2) (layer "F.Cu") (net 4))
 (segment (start 138.87 95.35) (end 142.73 95.35) (width 0.2) (layer "F.Cu") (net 4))
 (segment (start 122 117.06) (end 125.94 117.06) (width 0.2) (layer "F.Cu") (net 4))
 (segment (start 142.73 95.35) (end 144 94.08) (width 0.2) (layer "F.Cu") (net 4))
 (via (at 143.9 92.45) (size 0.6) (drill 0.3) (layers "F.Cu" "B.Cu") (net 4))
 (via (at 130.5 112.5) (size 0.6) (drill 0.3) (layers "F.Cu" "B.Cu") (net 4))
 (via (at 135.5 112.5) (size 0.6) (drill 0.3) (layers "F.Cu" "B.Cu") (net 4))
 (segment (start 143.9 91.14) (end 145.74 89.3) (width 0.2) (layer "B.Cu") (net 4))
 (segment (start 143.9 92.45) (end 143.9 91.14) (width 0.2) (layer "B.Cu") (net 4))
 (segment (start 130.5 112.5) (end 135.5 112.5) (width 0.2) (layer "B.Cu") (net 4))
 (segment (start 139.78 114.52) (end 141.34 114.52) (width 0.2) (layer "F.Cu") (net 20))
 (segment (start 144 106.28) (end 145.74 104.54) (width 0.2) (layer "F.Cu") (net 20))
 (segment (start 144 111.86) (end 144 106.28) (width 0.2) (layer "F.Cu") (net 20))
 (segment (start 141.34 114.52) (end 144 111.86) (width 0.2) (layer "F.Cu") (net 20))
 (segment (start 145.56 81.5) (end 145.74 81.68) (width 0.2) (layer "F.Cu") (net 24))
 (segment (start 139.78 81.5) (end 145.56 81.5) (width 0.2) (layer "F.Cu") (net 24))
 (segment (start 122 96.74) (end 130.32 96.74) (width 0.2) (layer "F.Cu") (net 14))
 (segment (start 130.32 96.74) (end 130.5 96.92) (width 0.2) (layer "F.Cu") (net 14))
 (segment (start 127.78 89.12) (end 130.5 91.84) (width 0.2) (layer "F.Cu") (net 12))
 (segment (start 122 89.12) (end 127.78 89.12) (width 0.2) (layer "F.Cu") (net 12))
 (segment (start 128.14 109.44) (end 130.5 107.08) (width 0.2) (layer "F.Cu") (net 18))
 (segment (start 122 109.44) (end 128.14 109.44) (width 0.2) (layer "F.Cu") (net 18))
 (segment (start 135 102.433654) (end 139.433654 98) (width 0.2) (layer "B.Cu") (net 1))
 (segment (start 139.433654 98) (end 141.492521 98) (width 0.2) (layer "B.Cu") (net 1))
 (segment (start 122 111.98) (end 126.98 111.98) (width 0.2) (layer "B.Cu") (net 1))
 (segment (start 126.98 111.98) (end 127 112) (width 0.2) (layer "B.Cu") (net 1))
 (segment (start 129.5 109.5) (end 135 109.5) (width 0.2) (layer "B.Cu") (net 1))
 (segment (start 135 109.5) (end 135 102.433654) (width 0.2) (layer "B.Cu") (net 1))
 (segment (start 141.492521 98) (end 142.572521 96.92) (width 0.2) (layer "B.Cu") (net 1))
 (segment (start 142.572521 96.92) (end 145.74 96.92) (width 0.2) (layer "B.Cu") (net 1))
 (segment (start 127 112) (end 129.5 109.5) (width 0.2) (layer "B.Cu") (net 1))
 (segment (start 134.5 121) (end 134.5 94.64) (width 0.2) (layer "F.Cu") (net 5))
 (segment (start 134.5 94.64) (end 138.6894 90.4506) (width 0.2) (layer "F.Cu") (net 5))
 (segment (start 133.5 122) (end 134.5 121) (width 0.2) (layer "F.Cu") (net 5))
 (segment (start 138.6894 90.4506) (end 142.8141 90.4506) (width 0.2) (layer "F.Cu") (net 5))
 (via (at 133.5 122) (size 0.6) (drill 0.3) (layers "F.Cu" "B.Cu") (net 5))
 (segment (start 122.275735 122.415735) (end 122 122.14) (width 0.2) (layer "B.Cu") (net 5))
 (segment (start 122 122.14) (end 133.36 122.14) (width 0.2) (layer "B.Cu") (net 5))
 (segment (start 133.36 122.14) (end 133.5 122) (width 0.2) (layer "B.Cu") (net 5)))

